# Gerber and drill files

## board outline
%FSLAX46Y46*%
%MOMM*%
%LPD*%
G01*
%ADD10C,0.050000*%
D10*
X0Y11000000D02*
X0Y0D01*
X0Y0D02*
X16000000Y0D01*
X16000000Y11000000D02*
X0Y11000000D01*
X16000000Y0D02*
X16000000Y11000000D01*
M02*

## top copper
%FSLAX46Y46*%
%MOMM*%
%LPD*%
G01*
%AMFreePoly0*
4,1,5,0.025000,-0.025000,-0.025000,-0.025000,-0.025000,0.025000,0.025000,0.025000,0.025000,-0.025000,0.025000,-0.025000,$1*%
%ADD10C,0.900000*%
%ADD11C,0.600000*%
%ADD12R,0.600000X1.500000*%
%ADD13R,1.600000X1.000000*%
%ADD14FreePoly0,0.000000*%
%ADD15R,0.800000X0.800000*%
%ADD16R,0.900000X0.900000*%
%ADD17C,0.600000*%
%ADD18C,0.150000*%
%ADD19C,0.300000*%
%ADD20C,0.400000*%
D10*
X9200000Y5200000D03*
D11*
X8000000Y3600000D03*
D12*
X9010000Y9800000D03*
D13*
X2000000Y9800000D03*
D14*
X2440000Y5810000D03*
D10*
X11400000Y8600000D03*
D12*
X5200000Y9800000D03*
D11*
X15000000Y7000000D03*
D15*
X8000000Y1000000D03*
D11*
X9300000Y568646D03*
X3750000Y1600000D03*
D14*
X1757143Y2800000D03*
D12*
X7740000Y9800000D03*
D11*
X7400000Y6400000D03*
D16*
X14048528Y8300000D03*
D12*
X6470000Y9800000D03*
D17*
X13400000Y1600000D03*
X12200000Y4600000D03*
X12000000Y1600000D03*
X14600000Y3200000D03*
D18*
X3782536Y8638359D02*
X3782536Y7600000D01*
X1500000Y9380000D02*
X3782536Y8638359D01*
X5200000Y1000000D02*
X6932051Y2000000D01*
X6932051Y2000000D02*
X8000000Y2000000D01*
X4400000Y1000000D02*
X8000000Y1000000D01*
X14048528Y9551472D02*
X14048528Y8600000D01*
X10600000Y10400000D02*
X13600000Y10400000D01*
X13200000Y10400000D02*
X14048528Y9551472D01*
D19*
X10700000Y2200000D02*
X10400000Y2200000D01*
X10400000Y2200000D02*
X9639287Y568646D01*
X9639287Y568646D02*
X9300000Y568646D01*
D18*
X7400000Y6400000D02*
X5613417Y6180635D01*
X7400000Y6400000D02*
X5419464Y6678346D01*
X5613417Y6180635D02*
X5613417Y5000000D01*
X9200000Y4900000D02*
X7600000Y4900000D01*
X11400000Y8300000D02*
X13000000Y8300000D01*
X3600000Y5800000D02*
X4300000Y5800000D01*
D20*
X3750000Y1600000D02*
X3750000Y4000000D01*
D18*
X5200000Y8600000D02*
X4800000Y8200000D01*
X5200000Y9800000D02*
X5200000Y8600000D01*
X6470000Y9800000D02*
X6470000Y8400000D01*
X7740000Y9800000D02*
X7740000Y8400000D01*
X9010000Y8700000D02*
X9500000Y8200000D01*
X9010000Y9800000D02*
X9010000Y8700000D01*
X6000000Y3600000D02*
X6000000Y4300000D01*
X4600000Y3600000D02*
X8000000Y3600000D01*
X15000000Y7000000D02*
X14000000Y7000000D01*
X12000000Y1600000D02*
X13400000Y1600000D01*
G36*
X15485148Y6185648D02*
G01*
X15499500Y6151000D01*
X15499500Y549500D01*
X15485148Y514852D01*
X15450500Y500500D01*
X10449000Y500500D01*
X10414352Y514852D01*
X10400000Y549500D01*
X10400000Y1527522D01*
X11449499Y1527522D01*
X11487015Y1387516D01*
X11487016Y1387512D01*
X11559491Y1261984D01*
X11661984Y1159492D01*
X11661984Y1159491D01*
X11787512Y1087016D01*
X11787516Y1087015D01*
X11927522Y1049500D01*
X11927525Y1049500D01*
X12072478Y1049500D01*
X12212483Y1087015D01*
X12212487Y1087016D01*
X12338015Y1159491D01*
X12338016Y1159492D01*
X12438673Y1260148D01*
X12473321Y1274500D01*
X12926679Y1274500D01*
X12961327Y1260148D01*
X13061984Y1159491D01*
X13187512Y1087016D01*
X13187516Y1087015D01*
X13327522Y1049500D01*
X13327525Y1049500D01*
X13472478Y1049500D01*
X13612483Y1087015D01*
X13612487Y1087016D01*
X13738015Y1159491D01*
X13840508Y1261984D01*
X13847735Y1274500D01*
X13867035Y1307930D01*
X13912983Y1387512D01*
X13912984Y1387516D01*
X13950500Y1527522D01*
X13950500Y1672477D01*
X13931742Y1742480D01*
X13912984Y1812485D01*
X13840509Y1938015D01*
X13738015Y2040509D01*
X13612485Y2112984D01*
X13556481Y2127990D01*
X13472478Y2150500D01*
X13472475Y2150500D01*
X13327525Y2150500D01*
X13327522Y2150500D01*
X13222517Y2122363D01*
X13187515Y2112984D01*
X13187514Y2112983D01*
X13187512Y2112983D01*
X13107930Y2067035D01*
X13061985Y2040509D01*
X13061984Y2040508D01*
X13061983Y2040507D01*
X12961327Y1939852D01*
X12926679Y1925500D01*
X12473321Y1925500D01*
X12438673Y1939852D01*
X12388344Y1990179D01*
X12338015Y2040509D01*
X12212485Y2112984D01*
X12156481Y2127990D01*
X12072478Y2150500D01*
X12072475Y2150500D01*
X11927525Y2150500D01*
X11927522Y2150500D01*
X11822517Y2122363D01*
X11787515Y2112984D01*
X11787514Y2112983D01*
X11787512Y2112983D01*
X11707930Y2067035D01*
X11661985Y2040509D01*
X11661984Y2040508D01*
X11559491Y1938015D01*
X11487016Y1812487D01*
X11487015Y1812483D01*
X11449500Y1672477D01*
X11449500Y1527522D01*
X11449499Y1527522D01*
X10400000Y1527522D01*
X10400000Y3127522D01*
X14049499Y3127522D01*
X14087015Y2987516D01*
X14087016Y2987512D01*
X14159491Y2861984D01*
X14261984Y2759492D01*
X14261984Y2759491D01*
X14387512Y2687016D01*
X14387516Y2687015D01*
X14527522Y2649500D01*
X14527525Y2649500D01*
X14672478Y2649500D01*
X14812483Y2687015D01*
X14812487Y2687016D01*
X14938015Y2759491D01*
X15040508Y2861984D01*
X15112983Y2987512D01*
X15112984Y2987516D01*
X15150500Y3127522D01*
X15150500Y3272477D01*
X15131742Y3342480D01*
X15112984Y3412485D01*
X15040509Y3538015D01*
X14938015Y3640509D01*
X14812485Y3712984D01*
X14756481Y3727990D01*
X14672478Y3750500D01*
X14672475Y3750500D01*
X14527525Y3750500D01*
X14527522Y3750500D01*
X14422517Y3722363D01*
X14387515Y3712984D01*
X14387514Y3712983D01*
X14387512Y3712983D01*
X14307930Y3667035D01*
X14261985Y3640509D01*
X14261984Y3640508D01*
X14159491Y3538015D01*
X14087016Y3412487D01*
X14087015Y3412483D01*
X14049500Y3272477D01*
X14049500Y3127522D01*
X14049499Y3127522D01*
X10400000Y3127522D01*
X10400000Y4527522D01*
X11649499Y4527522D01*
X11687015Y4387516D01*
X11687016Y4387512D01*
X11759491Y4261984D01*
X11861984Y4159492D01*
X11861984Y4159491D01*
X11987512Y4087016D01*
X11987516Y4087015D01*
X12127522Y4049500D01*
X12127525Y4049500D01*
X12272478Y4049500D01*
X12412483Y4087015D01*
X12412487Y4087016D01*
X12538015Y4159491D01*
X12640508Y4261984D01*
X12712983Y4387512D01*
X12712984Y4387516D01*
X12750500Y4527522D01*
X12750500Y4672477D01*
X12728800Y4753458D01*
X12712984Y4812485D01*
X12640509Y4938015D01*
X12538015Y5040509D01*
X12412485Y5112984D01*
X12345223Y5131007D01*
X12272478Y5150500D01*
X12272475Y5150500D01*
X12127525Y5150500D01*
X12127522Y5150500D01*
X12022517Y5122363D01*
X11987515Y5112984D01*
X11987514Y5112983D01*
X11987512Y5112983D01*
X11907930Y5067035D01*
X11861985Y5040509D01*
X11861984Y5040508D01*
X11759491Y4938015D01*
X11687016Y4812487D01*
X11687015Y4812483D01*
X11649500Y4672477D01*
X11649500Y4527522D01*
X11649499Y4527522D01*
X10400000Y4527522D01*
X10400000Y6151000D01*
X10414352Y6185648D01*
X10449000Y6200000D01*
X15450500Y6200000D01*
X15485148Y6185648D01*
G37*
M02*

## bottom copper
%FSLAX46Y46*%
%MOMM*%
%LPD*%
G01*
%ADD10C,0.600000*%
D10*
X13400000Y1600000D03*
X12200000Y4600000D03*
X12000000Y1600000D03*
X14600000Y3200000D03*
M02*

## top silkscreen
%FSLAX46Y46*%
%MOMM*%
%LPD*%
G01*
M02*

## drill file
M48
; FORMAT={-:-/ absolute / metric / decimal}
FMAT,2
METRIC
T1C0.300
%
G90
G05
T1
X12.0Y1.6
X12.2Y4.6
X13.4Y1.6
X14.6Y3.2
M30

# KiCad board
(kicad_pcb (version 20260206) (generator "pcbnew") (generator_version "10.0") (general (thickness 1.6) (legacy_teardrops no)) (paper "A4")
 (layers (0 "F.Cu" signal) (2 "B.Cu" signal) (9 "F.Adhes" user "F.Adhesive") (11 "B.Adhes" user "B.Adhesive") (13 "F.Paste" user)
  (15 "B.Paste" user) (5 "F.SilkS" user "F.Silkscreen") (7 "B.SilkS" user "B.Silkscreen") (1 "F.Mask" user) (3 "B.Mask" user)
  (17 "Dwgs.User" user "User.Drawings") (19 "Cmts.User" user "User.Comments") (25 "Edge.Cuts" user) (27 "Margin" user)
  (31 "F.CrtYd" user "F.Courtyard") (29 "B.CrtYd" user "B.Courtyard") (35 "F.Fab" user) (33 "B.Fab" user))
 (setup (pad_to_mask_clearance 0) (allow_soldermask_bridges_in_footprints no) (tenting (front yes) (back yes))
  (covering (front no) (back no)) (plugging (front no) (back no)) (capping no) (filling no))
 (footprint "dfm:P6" (layer "F.Cu") (at 9.2 -5.2)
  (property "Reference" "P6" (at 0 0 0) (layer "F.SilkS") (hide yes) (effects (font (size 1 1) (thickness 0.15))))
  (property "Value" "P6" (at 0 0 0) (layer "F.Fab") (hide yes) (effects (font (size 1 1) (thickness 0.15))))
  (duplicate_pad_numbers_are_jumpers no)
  (pad "1" smd circle (at 0 0) (size 0.9 0.9) (layers "F.Cu" "F.Mask" "F.Paste") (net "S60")))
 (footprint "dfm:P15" (layer "F.Cu") (at 8 -3.6)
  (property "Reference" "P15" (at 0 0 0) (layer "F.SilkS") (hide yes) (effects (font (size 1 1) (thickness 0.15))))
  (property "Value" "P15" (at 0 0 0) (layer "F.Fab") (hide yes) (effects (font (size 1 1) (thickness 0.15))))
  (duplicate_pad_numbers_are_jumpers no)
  (pad "1" smd circle (at 0 0) (size 0.6 0.6) (layers "F.Cu" "F.Mask" "F.Paste") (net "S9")))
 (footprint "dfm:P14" (layer "F.Cu") (at 9.01 -9.8)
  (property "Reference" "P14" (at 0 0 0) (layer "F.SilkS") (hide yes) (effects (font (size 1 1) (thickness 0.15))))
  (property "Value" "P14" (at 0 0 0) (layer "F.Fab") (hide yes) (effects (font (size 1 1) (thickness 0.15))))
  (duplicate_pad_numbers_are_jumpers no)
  (pad "1" smd rect (at 0 0) (size 0.6 1.5) (layers "F.Cu" "F.Mask" "F.Paste") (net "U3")))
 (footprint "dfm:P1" (layer "F.Cu") (at 2 -9.8)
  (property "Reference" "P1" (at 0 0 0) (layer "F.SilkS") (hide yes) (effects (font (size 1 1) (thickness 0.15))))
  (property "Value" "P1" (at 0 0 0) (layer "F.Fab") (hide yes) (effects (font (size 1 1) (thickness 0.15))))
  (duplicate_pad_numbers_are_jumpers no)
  (pad "1" smd rect (at 0 0) (size 1.6 1) (layers "F.Cu" "F.Mask" "F.Paste") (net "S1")))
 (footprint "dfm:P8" (layer "F.Cu") (at 2.44 -5.81)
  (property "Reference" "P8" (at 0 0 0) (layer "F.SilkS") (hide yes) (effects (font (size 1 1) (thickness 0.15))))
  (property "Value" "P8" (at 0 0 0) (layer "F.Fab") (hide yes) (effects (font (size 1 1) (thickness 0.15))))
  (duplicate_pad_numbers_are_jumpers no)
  (pad "1" smd custom (at 0 0) (size 0.05 0.05) (layers "F.Cu" "F.Mask" "F.Paste") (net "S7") (options (clearance outline) (anchor rect))
   (primitives)))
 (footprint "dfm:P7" (layer "F.Cu") (at 11.4 -8.6)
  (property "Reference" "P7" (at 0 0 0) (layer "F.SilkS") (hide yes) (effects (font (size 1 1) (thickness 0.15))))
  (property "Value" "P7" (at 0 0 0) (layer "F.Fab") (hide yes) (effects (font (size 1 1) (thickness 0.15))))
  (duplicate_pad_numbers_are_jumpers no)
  (pad "1" smd circle (at 0 0) (size 0.9 0.9) (layers "F.Cu" "F.Mask" "F.Paste") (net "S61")))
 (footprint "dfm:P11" (layer "F.Cu") (at 5.2 -9.8)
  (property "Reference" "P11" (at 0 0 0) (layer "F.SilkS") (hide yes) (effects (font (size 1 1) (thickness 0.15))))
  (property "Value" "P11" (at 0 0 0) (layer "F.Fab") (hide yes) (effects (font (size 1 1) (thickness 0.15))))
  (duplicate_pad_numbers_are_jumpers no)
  (pad "1" smd rect (at 0 0) (size 0.6 1.5) (layers "F.Cu" "F.Mask" "F.Paste") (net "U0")))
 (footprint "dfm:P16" (layer "F.Cu") (at 15 -7)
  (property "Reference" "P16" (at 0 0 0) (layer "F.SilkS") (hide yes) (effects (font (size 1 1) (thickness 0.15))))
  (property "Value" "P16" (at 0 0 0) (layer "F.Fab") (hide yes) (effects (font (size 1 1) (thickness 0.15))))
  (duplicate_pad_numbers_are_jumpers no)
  (pad "1" smd circle (at 0 0) (size 0.6 0.6) (layers "F.Cu" "F.Mask" "F.Paste") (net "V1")))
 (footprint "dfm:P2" (layer "F.Cu") (at 8 -1)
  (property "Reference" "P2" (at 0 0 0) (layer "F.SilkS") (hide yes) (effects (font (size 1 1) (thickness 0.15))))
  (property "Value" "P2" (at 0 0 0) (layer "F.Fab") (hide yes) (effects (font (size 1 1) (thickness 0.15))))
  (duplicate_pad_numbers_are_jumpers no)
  (pad "1" smd rect (at 0 0) (size 0.8 0.8) (layers "F.Cu" "F.Mask" "F.Paste") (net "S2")))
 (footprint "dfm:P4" (layer "F.Cu") (at 9.3 -0.568646)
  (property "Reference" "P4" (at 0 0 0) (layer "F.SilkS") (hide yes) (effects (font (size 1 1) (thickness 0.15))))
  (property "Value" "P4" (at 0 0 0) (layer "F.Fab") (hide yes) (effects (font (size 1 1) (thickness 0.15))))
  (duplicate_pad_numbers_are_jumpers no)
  (pad "1" smd circle (at 0 0) (size 0.6 0.6) (layers "F.Cu" "F.Mask" "F.Paste") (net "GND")))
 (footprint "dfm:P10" (layer "F.Cu") (at 3.75 -1.6)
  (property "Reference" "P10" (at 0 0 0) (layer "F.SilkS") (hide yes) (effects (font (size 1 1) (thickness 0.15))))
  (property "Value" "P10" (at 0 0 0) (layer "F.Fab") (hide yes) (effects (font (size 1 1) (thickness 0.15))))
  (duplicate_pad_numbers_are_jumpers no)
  (pad "1" smd circle (at 0 0) (size 0.6 0.6) (layers "F.Cu" "F.Mask" "F.Paste") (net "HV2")))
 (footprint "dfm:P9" (layer "F.Cu") (at 1.757143 -2.8)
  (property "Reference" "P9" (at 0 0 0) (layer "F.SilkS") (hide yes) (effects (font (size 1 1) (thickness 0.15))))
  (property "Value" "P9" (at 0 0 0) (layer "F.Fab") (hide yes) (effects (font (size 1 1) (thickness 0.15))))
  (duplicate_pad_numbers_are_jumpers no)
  (pad "1" smd custom (at 0 0) (size 0.05 0.05) (layers "F.Cu" "F.Mask" "F.Paste") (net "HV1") (options (clearance outline) (anchor rect))
   (primitives)))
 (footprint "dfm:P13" (layer "F.Cu") (at 7.74 -9.8)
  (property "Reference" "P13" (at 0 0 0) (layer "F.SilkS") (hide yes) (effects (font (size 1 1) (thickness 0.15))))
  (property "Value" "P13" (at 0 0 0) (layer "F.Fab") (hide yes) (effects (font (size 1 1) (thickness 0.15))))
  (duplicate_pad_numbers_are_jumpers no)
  (pad "1" smd rect (at 0 0) (size 0.6 1.5) (layers "F.Cu" "F.Mask" "F.Paste") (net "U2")))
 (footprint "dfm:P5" (layer "F.Cu") (at 7.4 -6.4)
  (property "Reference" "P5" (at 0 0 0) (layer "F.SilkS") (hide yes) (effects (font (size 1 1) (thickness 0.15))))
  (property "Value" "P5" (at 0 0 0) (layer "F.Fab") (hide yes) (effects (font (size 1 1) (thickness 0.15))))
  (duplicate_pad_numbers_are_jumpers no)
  (pad "1" smd circle (at 0 0) (size 0.6 0.6) (layers "F.Cu" "F.Mask" "F.Paste") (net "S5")))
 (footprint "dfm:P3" (layer "F.Cu") (at 14.048528 -8.3)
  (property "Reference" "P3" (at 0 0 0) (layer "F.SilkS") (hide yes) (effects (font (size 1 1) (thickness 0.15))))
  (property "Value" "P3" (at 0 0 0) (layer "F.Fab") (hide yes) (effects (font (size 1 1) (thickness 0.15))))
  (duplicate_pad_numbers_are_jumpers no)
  (pad "1" smd rect (at 0 0) (size 0.9 0.9) (layers "F.Cu" "F.Mask" "F.Paste") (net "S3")))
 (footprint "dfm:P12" (layer "F.Cu") (at 6.47 -9.8)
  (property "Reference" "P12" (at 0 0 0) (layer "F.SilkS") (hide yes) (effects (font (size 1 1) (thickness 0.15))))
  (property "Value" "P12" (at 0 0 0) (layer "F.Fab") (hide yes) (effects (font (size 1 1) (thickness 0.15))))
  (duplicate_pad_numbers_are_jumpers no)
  (pad "1" smd rect (at 0 0) (size 0.6 1.5) (layers "F.Cu" "F.Mask" "F.Paste") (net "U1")))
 (gr_line (start 0 -11) (end 0 0) (stroke (width 0.05) (type solid)) (layer "Edge.Cuts"))
 (gr_line (start 0 0) (end 16 0) (stroke (width 0.05) (type solid)) (layer "Edge.Cuts"))
 (gr_line (start 16 -11) (end 0 -11) (stroke (width 0.05) (type solid)) (layer "Edge.Cuts"))
 (gr_line (start 16 0) (end 16 -11) (stroke (width 0.05) (type solid)) (layer "Edge.Cuts"))
 (segment (start 3.782536 -8.638359) (end 3.782536 -7.6) (width 0.15) (layer "F.Cu") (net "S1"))
 (segment (start 1.5 -9.38) (end 3.782536 -8.638359) (width 0.15) (layer "F.Cu") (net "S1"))
 (segment (start 5.2 -1) (end 6.932051 -2) (width 0.15) (layer "F.Cu") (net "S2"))
 (segment (start 6.932051 -2) (end 8 -2) (width 0.15) (layer "F.Cu") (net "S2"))
 (segment (start 4.4 -1) (end 8 -1) (width 0.15) (layer "F.Cu") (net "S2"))
 (segment (start 14.048528 -9.551472) (end 14.048528 -8.6) (width 0.15) (layer "F.Cu") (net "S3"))
 (segment (start 10.6 -10.4) (end 13.6 -10.4) (width 0.15) (layer "F.Cu") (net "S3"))
 (segment (start 13.2 -10.4) (end 14.048528 -9.551472) (width 0.15) (layer "F.Cu") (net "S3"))
 (segment (start 10.7 -2.2) (end 10.4 -2.2) (width 0.3) (layer "F.Cu") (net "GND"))
 (segment (start 10.4 -2.2) (end 9.639287 -0.568646) (width 0.3) (layer "F.Cu") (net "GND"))
 (segment (start 9.639287 -0.568646) (end 9.3 -0.568646) (width 0.3) (layer "F.Cu") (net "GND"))
 (segment (start 7.4 -6.4) (end 5.613417 -6.180635) (width 0.15) (layer "F.Cu") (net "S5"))
 (segment (start 7.4 -6.4) (end 5.419464 -6.678346) (width 0.15) (layer "F.Cu") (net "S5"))
 (segment (start 5.613417 -6.180635) (end 5.613417 -5) (width 0.15) (layer "F.Cu") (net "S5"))
 (segment (start 9.2 -4.9) (end 7.6 -4.9) (width 0.15) (layer "F.Cu") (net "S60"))
 (segment (start 11.4 -8.3) (end 13 -8.3) (width 0.15) (layer "F.Cu") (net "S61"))
 (segment (start 3.6 -5.8) (end 4.3 -5.8) (width 0.15) (layer "F.Cu") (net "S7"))
 (segment (start 3.75 -1.6) (end 3.75 -4) (width 0.4) (layer "F.Cu") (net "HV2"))
 (segment (start 5.2 -8.6) (end 4.8 -8.2) (width 0.15) (layer "F.Cu") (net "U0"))
 (segment (start 5.2 -9.8) (end 5.2 -8.6) (width 0.15) (layer "F.Cu") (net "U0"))
 (segment (start 6.47 -9.8) (end 6.47 -8.4) (width 0.15) (layer "F.Cu") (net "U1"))
 (segment (start 7.74 -9.8) (end 7.74 -8.4) (width 0.15) (layer "F.Cu") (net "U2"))
 (segment (start 9.01 -8.7) (end 9.5 -8.2) (width 0.15) (layer "F.Cu") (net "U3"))
 (segment (start 9.01 -9.8) (end 9.01 -8.7) (width 0.15) (layer "F.Cu") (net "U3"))
 (segment (start 6 -3.6) (end 6 -4.3) (width 0.15) (layer "F.Cu") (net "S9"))
 (segment (start 4.6 -3.6) (end 8 -3.6) (width 0.15) (layer "F.Cu") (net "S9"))
 (segment (start 15 -7) (end 14 -7) (width 0.15) (layer "F.Cu") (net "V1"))
 (segment (start 12 -1.6) (end 13.4 -1.6) (width 0.15) (layer "F.Cu") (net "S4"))
 (via (at 13.4 -1.6) (size 0.6) (drill 0.3) (layers "F.Cu" "B.Cu") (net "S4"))
 (via (at 12.2 -4.6) (size 0.6) (drill 0.3) (layers "F.Cu" "B.Cu") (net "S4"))
 (via (at 12 -1.6) (size 0.6) (drill 0.3) (layers "F.Cu" "B.Cu") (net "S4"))
 (via (at 14.6 -3.2) (size 0.6) (drill 0.3) (layers "F.Cu" "B.Cu") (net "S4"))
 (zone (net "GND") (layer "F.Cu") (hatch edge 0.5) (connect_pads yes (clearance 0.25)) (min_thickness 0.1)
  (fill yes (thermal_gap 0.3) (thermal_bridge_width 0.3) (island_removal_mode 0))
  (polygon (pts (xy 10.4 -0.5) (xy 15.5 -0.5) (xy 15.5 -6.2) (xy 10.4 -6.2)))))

